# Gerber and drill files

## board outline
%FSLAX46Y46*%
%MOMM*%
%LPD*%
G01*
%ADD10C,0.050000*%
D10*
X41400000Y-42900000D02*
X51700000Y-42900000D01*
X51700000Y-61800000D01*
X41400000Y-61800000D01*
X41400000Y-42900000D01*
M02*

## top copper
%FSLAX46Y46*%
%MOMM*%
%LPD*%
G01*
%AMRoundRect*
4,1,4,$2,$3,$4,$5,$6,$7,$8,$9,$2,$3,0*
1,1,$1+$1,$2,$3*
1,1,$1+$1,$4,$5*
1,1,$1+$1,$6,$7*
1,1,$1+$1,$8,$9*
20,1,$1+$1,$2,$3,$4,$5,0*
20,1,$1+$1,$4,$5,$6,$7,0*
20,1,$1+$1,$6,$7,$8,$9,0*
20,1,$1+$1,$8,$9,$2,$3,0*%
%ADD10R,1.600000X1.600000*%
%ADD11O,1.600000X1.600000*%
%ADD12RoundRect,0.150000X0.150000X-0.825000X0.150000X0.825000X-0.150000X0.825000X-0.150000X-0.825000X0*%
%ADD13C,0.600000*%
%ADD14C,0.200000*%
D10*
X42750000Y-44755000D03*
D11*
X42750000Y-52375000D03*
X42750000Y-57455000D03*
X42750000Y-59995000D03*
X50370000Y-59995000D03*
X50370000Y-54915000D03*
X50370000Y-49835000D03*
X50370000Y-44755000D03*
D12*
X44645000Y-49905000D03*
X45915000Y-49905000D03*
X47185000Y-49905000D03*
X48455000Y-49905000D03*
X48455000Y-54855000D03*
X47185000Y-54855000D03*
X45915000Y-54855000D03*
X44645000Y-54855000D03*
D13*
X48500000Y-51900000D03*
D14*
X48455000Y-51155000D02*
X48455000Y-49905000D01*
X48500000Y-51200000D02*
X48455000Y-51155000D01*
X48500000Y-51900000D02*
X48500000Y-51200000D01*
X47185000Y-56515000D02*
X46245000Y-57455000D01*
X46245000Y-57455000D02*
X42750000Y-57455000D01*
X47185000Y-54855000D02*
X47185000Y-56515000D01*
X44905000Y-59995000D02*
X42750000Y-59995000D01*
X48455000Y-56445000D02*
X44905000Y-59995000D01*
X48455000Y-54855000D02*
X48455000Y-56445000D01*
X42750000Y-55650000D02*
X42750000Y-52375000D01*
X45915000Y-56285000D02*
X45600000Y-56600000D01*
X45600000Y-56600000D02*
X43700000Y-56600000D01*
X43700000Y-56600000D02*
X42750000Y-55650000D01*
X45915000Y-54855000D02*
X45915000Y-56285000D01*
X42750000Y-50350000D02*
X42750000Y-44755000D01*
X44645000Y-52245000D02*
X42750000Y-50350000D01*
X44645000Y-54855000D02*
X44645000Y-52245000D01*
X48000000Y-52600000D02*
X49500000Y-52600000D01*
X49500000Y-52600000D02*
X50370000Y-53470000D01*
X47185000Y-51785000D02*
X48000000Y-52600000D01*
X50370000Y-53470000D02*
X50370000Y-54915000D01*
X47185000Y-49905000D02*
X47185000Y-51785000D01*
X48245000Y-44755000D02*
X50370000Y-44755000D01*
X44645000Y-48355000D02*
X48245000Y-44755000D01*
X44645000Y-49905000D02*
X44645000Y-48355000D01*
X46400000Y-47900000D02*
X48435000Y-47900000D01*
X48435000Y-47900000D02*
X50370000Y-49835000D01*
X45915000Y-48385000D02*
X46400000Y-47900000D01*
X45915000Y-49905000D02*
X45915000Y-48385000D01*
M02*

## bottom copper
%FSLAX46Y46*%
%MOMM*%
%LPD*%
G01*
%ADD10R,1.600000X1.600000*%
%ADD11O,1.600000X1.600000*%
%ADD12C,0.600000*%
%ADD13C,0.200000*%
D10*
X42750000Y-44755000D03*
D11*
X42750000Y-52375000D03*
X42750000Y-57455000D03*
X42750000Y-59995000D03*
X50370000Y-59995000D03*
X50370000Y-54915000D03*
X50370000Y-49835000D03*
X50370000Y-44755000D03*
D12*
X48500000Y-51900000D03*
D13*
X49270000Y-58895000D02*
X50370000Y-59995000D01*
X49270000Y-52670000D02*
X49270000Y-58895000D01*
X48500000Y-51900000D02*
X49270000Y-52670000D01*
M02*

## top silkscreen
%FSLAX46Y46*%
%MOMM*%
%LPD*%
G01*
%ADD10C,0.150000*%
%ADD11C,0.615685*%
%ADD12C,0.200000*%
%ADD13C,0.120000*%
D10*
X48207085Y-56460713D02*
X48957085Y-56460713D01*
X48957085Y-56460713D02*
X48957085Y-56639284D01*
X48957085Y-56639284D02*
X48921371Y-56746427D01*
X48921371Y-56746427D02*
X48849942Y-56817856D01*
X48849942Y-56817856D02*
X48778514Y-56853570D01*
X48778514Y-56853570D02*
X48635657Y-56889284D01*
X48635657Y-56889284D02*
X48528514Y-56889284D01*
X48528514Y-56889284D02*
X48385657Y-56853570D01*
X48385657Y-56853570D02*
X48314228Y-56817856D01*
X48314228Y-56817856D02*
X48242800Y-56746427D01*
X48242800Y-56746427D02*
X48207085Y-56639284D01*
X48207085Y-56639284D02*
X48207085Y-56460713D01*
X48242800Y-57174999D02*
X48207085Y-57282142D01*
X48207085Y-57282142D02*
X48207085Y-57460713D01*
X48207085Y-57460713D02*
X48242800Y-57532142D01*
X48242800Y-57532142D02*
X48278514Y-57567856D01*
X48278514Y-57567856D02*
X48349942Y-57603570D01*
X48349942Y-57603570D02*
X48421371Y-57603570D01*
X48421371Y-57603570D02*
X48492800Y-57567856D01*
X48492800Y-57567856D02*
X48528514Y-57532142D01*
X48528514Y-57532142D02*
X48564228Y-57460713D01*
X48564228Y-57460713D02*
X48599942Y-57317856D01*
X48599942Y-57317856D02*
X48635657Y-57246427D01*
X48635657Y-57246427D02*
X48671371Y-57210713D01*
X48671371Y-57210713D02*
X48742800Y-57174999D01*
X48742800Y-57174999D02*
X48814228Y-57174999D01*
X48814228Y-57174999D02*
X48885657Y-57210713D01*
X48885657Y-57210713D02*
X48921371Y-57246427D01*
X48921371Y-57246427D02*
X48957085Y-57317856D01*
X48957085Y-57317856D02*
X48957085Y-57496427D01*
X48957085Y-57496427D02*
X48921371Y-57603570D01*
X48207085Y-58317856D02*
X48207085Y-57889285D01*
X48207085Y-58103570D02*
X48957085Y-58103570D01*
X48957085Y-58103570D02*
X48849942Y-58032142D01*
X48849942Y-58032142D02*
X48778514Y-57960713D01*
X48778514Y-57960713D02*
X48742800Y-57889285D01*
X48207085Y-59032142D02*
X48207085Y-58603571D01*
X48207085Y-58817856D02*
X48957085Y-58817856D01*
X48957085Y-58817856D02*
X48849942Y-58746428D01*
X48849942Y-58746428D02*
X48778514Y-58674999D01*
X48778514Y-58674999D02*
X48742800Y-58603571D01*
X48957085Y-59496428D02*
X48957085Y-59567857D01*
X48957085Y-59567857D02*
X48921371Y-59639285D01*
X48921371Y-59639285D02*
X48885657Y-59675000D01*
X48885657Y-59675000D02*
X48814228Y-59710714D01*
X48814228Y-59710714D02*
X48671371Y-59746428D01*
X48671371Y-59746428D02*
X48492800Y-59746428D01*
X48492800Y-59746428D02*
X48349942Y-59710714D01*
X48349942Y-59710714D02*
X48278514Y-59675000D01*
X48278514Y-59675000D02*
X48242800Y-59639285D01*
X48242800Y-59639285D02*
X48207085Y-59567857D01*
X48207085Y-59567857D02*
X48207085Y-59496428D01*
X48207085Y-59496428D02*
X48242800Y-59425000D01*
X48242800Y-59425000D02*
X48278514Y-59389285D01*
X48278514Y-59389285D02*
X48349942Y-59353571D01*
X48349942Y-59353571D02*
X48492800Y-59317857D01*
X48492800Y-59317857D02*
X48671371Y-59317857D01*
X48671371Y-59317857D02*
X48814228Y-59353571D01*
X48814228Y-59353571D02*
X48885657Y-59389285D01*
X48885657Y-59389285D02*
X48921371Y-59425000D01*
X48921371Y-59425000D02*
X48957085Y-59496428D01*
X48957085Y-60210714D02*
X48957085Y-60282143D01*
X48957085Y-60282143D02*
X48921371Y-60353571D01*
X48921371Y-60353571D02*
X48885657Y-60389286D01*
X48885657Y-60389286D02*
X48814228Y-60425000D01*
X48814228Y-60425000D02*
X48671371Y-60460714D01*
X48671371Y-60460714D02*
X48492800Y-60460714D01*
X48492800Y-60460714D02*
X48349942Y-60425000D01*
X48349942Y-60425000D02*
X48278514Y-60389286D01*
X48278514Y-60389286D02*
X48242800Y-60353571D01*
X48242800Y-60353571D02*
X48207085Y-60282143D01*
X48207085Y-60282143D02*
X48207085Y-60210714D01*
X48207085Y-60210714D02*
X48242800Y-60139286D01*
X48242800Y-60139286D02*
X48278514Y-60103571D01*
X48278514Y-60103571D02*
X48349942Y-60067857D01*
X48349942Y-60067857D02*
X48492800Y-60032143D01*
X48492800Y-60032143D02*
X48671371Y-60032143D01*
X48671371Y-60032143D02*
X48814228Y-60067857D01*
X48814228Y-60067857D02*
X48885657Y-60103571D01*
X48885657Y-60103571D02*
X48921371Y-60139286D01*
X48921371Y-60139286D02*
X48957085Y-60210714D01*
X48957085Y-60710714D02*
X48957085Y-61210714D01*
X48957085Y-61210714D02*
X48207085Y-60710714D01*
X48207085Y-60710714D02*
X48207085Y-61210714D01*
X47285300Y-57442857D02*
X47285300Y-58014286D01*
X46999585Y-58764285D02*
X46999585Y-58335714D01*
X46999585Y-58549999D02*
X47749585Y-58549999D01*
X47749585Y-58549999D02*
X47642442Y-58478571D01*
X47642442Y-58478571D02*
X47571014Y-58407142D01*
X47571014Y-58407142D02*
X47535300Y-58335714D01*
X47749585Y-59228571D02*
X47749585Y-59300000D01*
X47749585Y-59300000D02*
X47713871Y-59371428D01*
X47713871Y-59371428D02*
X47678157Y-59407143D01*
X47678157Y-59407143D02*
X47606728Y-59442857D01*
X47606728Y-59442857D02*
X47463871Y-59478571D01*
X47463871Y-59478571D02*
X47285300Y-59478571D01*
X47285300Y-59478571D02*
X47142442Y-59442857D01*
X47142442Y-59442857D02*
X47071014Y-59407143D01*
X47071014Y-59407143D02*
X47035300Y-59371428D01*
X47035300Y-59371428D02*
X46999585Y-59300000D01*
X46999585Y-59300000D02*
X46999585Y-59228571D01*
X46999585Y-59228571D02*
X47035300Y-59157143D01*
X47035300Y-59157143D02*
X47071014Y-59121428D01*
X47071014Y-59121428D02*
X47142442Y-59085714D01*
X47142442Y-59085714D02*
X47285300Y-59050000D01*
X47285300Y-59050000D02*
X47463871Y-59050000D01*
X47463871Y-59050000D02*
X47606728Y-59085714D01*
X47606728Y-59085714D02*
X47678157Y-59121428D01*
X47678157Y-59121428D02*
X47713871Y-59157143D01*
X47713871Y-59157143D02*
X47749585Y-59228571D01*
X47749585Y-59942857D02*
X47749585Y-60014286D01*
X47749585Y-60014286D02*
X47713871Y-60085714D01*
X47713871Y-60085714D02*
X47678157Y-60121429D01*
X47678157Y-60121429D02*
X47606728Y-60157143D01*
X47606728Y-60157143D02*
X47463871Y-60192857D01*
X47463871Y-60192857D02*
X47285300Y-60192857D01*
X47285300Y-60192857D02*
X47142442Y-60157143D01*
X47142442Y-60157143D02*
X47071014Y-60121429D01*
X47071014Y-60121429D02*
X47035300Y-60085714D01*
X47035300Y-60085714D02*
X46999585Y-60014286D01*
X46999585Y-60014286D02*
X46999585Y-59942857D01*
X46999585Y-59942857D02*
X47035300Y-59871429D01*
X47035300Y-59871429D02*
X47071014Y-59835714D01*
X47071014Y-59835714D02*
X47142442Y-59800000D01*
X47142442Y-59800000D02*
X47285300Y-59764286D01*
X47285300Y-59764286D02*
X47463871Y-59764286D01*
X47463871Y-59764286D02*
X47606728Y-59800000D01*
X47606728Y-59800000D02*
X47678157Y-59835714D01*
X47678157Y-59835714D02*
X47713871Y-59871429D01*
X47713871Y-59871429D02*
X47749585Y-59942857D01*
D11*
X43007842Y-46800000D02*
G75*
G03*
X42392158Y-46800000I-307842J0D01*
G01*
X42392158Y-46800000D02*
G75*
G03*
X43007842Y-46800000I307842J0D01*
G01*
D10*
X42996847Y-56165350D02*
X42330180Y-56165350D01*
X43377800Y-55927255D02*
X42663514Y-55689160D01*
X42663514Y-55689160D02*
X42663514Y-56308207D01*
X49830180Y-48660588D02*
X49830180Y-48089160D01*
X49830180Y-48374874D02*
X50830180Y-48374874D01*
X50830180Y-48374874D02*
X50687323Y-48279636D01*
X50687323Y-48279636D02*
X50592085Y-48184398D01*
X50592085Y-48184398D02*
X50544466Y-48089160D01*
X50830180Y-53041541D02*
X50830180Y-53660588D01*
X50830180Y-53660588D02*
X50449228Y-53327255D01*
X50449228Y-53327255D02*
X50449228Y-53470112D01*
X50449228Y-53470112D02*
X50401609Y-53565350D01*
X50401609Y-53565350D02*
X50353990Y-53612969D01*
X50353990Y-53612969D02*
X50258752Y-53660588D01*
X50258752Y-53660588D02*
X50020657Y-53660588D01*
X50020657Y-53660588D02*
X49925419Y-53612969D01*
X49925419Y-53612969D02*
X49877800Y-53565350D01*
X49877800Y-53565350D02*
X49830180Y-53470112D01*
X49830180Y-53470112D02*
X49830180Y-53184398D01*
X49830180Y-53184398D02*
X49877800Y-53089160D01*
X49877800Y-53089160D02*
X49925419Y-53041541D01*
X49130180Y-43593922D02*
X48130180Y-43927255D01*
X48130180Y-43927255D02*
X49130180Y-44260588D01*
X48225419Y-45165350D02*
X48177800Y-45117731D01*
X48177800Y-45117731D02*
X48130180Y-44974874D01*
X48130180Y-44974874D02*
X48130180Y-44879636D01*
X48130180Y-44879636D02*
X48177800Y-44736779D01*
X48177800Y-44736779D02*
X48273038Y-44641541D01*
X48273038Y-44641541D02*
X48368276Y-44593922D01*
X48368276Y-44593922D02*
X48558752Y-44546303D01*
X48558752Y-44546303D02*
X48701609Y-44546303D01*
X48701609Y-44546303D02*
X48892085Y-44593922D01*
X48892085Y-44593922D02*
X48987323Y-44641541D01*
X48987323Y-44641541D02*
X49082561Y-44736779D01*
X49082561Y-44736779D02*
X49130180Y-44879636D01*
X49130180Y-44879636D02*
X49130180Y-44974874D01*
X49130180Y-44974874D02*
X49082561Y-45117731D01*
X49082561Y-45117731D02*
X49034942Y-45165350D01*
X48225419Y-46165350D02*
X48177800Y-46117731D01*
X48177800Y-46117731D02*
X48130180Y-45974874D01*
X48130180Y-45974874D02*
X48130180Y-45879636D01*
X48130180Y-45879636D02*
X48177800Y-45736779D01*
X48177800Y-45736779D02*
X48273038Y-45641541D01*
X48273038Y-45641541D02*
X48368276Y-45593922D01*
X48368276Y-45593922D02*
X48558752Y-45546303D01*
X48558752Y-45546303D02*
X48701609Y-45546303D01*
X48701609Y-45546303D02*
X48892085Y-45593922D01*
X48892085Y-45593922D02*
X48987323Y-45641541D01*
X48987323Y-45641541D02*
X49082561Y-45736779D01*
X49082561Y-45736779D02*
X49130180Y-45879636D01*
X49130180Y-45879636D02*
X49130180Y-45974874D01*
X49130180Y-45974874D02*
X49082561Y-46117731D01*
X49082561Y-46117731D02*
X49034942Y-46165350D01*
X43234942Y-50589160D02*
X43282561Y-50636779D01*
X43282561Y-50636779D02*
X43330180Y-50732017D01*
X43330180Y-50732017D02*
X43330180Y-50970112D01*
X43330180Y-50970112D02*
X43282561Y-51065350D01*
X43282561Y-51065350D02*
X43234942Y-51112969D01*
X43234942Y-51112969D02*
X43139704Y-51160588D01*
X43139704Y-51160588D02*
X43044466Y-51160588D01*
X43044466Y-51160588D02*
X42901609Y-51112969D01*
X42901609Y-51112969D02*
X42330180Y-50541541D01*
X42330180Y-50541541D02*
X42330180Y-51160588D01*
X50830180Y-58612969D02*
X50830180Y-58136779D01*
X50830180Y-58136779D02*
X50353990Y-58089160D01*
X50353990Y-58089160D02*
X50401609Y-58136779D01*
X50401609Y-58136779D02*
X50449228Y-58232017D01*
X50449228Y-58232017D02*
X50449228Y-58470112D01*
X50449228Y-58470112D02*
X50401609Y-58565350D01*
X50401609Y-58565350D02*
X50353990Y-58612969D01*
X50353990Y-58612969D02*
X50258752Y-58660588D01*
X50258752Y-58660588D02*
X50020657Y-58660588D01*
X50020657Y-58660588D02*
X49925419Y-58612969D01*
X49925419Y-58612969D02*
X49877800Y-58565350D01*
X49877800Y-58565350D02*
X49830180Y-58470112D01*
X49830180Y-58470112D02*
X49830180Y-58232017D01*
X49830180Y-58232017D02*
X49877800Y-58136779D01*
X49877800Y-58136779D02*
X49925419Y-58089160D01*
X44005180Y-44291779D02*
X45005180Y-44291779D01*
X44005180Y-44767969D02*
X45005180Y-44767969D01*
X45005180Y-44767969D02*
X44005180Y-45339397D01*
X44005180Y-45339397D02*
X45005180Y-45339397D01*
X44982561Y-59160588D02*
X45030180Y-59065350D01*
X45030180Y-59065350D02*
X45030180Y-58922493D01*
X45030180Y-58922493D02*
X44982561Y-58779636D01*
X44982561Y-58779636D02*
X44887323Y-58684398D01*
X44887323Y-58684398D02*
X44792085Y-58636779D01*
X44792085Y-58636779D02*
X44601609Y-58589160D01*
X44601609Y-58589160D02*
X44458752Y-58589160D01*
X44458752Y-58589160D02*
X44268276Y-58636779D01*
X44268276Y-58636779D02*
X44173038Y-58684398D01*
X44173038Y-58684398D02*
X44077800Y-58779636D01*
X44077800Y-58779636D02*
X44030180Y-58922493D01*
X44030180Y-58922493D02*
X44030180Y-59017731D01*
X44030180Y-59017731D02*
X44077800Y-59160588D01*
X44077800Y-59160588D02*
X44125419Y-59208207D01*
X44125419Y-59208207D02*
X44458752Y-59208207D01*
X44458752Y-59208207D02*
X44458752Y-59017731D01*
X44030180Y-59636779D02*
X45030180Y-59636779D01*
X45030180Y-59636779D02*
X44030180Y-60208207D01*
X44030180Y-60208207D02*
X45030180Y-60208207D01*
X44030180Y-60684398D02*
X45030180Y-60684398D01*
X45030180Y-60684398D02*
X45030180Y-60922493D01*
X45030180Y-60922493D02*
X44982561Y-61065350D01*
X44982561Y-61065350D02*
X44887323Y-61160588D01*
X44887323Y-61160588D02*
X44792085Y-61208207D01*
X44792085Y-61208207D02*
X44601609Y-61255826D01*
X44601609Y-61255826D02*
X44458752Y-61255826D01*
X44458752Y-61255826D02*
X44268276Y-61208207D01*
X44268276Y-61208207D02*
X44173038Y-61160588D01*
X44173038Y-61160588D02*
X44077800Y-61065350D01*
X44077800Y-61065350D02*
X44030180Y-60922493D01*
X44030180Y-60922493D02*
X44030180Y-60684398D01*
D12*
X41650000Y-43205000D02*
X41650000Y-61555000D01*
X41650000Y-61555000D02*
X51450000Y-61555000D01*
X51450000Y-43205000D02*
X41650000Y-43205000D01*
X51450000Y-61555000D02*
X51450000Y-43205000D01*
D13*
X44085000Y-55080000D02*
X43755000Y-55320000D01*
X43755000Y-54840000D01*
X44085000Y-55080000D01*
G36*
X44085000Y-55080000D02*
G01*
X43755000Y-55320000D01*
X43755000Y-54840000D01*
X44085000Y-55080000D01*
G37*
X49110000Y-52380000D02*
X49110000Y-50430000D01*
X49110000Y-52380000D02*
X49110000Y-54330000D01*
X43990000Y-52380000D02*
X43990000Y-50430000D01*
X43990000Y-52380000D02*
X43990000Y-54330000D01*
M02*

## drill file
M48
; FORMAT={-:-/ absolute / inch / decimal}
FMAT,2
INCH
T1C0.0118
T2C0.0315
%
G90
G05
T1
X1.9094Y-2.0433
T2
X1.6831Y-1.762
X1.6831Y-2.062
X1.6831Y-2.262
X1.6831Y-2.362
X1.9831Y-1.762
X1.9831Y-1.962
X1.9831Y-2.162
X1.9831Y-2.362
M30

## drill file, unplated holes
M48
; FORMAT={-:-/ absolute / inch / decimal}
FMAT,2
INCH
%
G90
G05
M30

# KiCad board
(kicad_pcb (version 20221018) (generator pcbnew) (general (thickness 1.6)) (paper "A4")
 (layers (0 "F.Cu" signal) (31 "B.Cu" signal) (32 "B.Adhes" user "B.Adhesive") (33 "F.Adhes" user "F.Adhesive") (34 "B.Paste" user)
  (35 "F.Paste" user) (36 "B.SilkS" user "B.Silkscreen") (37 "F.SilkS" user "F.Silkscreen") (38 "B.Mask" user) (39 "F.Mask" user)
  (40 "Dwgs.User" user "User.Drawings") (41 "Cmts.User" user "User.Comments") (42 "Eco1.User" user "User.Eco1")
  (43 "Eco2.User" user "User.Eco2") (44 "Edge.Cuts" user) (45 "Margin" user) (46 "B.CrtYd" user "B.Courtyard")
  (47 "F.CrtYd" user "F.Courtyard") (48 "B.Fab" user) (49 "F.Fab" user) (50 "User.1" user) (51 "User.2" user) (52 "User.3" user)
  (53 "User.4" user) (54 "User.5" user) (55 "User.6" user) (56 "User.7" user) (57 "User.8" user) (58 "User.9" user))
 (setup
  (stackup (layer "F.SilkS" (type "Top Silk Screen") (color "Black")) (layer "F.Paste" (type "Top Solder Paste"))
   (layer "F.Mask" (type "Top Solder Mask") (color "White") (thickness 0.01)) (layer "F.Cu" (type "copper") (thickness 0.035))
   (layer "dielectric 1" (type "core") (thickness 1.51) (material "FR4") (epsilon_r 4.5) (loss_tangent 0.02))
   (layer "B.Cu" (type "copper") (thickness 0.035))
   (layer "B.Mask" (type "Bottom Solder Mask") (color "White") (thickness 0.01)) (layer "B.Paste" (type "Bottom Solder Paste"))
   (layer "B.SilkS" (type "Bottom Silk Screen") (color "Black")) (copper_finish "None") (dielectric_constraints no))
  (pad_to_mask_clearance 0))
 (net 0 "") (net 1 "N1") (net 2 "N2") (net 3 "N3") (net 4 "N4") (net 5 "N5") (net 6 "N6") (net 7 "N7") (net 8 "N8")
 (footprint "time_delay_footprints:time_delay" (layer "F.Cu") (at 42.75 44.755)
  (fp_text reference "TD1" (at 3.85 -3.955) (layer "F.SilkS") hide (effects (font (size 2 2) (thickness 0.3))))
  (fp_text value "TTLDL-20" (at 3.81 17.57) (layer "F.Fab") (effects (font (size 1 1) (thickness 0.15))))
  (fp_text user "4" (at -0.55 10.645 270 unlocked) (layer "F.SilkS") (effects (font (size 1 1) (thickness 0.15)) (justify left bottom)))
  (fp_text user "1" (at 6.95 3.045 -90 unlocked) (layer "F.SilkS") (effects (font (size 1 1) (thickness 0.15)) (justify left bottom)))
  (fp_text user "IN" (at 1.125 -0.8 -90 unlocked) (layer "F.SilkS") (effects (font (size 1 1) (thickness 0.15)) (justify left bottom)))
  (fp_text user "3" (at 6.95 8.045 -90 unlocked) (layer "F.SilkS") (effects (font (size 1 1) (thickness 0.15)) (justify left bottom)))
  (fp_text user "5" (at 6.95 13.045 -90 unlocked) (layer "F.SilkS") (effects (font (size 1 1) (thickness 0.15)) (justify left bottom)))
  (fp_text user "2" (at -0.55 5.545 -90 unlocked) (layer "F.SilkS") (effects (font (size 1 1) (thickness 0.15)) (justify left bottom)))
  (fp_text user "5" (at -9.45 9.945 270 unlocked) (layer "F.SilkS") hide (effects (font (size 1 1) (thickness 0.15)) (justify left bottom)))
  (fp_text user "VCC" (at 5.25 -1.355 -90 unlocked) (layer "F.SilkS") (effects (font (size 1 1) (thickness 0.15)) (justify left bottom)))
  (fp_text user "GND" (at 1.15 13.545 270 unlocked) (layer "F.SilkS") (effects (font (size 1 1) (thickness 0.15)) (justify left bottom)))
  (fp_line (start -1.1 -1.55) (end -1.1 16.8) (stroke (width 0.2) (type solid)) (layer "F.SilkS"))
  (fp_line (start -1.1 16.8) (end 8.7 16.8) (stroke (width 0.2) (type solid)) (layer "F.SilkS"))
  (fp_line (start 8.7 -1.55) (end -1.1 -1.55) (stroke (width 0.2) (type solid)) (layer "F.SilkS"))
  (fp_line (start 8.7 16.8) (end 8.7 -1.55) (stroke (width 0.2) (type solid)) (layer "F.SilkS"))
  (pad "1" thru_hole rect (at 0 0) (size 1.6 1.6) (drill 0.8) (layers "*.Cu" "*.Mask") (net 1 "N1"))
  (pad "4" thru_hole oval (at 0 7.62) (size 1.6 1.6) (drill 0.8) (layers "*.Cu" "*.Mask") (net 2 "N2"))
  (pad "6" thru_hole oval (at 0 12.7) (size 1.6 1.6) (drill 0.8) (layers "*.Cu" "*.Mask") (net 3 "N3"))
  (pad "7" thru_hole oval (at 0 15.24) (size 1.6 1.6) (drill 0.8) (layers "*.Cu" "*.Mask") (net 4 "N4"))
  (pad "8" thru_hole oval (at 7.62 15.24) (size 1.6 1.6) (drill 0.8) (layers "*.Cu" "*.Mask") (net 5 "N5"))
  (pad "10" thru_hole oval (at 7.62 10.16) (size 1.6 1.6) (drill 0.8) (layers "*.Cu" "*.Mask") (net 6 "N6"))
  (pad "12" thru_hole oval (at 7.62 5.08) (size 1.6 1.6) (drill 0.8) (layers "*.Cu" "*.Mask") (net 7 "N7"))
  (pad "14" thru_hole oval (at 7.62 0) (size 1.6 1.6) (drill 0.8) (layers "*.Cu" "*.Mask") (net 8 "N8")))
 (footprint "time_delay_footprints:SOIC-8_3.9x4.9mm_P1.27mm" (layer "F.Cu") (at 46.55 52.38 90)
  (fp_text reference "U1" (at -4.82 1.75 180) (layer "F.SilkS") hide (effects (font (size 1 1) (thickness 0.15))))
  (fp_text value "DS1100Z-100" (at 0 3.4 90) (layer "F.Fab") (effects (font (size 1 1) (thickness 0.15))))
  (fp_line (start 0 -2.56) (end -1.95 -2.56) (stroke (width 0.12) (type solid)) (layer "F.SilkS"))
  (fp_line (start 0 -2.56) (end 1.95 -2.56) (stroke (width 0.12) (type solid)) (layer "F.SilkS"))
  (fp_line (start 0 2.56) (end -1.95 2.56) (stroke (width 0.12) (type solid)) (layer "F.SilkS"))
  (fp_line (start 0 2.56) (end 1.95 2.56) (stroke (width 0.12) (type solid)) (layer "F.SilkS"))
  (fp_poly
   (pts (xy -2.7 -2.465) (xy -2.94 -2.795) (xy -2.46 -2.795) (xy -2.7 -2.465)) (stroke (width 0.12) (type solid)) (fill solid)
   (layer "F.SilkS"))
  (pad "1" smd roundrect (at -2.475 -1.905 90) (size 1.95 0.6) (layers "F.Cu" "F.Paste" "F.Mask") (roundrect_rratio 0.25) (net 1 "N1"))
  (pad "2" smd roundrect (at -2.475 -0.635 90) (size 1.95 0.6) (layers "F.Cu" "F.Paste" "F.Mask") (roundrect_rratio 0.25) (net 2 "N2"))
  (pad "3" smd roundrect (at -2.475 0.635 90) (size 1.95 0.6) (layers "F.Cu" "F.Paste" "F.Mask") (roundrect_rratio 0.25) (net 3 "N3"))
  (pad "4" smd roundrect (at -2.475 1.905 90) (size 1.95 0.6) (layers "F.Cu" "F.Paste" "F.Mask") (roundrect_rratio 0.25) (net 4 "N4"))
  (pad "5" smd roundrect (at 2.475 1.905 90) (size 1.95 0.6) (layers "F.Cu" "F.Paste" "F.Mask") (roundrect_rratio 0.25) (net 5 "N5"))
  (pad "6" smd roundrect (at 2.475 0.635 90) (size 1.95 0.6) (layers "F.Cu" "F.Paste" "F.Mask") (roundrect_rratio 0.25) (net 6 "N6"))
  (pad "7" smd roundrect (at 2.475 -0.635 90) (size 1.95 0.6) (layers "F.Cu" "F.Paste" "F.Mask") (roundrect_rratio 0.25) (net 7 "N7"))
  (pad "8" smd roundrect (at 2.475 -1.905 90) (size 1.95 0.6) (layers "F.Cu" "F.Paste" "F.Mask") (roundrect_rratio 0.25) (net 8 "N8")))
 (gr_circle (center 42.7 46.8) (end 43.265685 46.8) (stroke (width 0.1) (type solid)) (fill solid) (layer "F.SilkS"))
 (gr_rect (start 41.4 42.9) (end 51.7 61.8) (stroke (width 0.05) (type default)) (fill none) (layer "Edge.Cuts"))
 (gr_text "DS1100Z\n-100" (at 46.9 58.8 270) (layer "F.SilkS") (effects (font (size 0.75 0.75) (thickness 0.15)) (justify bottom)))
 (segment (start 42.75 50.35) (end 42.75 44.755) (width 0.2) (layer "F.Cu") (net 1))
 (segment (start 44.645 52.245) (end 42.75 50.35) (width 0.2) (layer "F.Cu") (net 1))
 (segment (start 44.645 54.855) (end 44.645 52.245) (width 0.2) (layer "F.Cu") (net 1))
 (segment (start 45.915 56.285) (end 45.6 56.6) (width 0.2) (layer "F.Cu") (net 2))
 (segment (start 45.915 54.855) (end 45.915 56.285) (width 0.2) (layer "F.Cu") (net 2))
 (segment (start 45.6 56.6) (end 43.7 56.6) (width 0.2) (layer "F.Cu") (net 2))
 (segment (start 42.75 55.65) (end 42.75 52.375) (width 0.2) (layer "F.Cu") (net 2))
 (segment (start 43.7 56.6) (end 42.75 55.65) (width 0.2) (layer "F.Cu") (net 2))
 (segment (start 46.245 57.455) (end 42.75 57.455) (width 0.2) (layer "F.Cu") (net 3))
 (segment (start 47.185 54.855) (end 47.185 56.515) (width 0.2) (layer "F.Cu") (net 3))
 (segment (start 47.185 56.515) (end 46.245 57.455) (width 0.2) (layer "F.Cu") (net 3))
 (segment (start 44.905 59.995) (end 42.75 59.995) (width 0.2) (layer "F.Cu") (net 4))
 (segment (start 48.455 54.855) (end 48.455 56.445) (width 0.2) (layer "F.Cu") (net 4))
 (segment (start 48.455 56.445) (end 44.905 59.995) (width 0.2) (layer "F.Cu") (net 4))
 (segment (start 48.5 51.2) (end 48.455 51.155) (width 0.2) (layer "F.Cu") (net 5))
 (segment (start 48.5 51.9) (end 48.5 51.2) (width 0.2) (layer "F.Cu") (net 5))
 (segment (start 48.455 51.155) (end 48.455 49.905) (width 0.2) (layer "F.Cu") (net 5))
 (via (at 48.5 51.9) (size 0.6) (drill 0.3) (layers "F.Cu" "B.Cu") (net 5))
 (segment (start 49.27 52.67) (end 49.27 58.895) (width 0.2) (layer "B.Cu") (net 5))
 (segment (start 49.27 58.895) (end 50.37 59.995) (width 0.2) (layer "B.Cu") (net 5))
 (segment (start 48.5 51.9) (end 49.27 52.67) (width 0.2) (layer "B.Cu") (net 5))
 (segment (start 50.37 53.47) (end 50.37 54.915) (width 0.2) (layer "F.Cu") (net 6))
 (segment (start 48 52.6) (end 49.5 52.6) (width 0.2) (layer "F.Cu") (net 6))
 (segment (start 47.185 51.785) (end 48 52.6) (width 0.2) (layer "F.Cu") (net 6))
 (segment (start 49.5 52.6) (end 50.37 53.47) (width 0.2) (layer "F.Cu") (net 6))
 (segment (start 47.185 49.905) (end 47.185 51.785) (width 0.2) (layer "F.Cu") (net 6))
 (segment (start 45.915 48.385) (end 46.4 47.9) (width 0.2) (layer "F.Cu") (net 7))
 (segment (start 45.915 49.905) (end 45.915 48.385) (width 0.2) (layer "F.Cu") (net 7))
 (segment (start 46.4 47.9) (end 48.435 47.9) (width 0.2) (layer "F.Cu") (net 7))
 (segment (start 48.435 47.9) (end 50.37 49.835) (width 0.2) (layer "F.Cu") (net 7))
 (segment (start 44.645 49.905) (end 44.645 48.355) (width 0.2) (layer "F.Cu") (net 8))
 (segment (start 44.645 48.355) (end 48.245 44.755) (width 0.2) (layer "F.Cu") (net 8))
 (segment (start 48.245 44.755) (end 50.37 44.755) (width 0.2) (layer "F.Cu") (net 8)))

